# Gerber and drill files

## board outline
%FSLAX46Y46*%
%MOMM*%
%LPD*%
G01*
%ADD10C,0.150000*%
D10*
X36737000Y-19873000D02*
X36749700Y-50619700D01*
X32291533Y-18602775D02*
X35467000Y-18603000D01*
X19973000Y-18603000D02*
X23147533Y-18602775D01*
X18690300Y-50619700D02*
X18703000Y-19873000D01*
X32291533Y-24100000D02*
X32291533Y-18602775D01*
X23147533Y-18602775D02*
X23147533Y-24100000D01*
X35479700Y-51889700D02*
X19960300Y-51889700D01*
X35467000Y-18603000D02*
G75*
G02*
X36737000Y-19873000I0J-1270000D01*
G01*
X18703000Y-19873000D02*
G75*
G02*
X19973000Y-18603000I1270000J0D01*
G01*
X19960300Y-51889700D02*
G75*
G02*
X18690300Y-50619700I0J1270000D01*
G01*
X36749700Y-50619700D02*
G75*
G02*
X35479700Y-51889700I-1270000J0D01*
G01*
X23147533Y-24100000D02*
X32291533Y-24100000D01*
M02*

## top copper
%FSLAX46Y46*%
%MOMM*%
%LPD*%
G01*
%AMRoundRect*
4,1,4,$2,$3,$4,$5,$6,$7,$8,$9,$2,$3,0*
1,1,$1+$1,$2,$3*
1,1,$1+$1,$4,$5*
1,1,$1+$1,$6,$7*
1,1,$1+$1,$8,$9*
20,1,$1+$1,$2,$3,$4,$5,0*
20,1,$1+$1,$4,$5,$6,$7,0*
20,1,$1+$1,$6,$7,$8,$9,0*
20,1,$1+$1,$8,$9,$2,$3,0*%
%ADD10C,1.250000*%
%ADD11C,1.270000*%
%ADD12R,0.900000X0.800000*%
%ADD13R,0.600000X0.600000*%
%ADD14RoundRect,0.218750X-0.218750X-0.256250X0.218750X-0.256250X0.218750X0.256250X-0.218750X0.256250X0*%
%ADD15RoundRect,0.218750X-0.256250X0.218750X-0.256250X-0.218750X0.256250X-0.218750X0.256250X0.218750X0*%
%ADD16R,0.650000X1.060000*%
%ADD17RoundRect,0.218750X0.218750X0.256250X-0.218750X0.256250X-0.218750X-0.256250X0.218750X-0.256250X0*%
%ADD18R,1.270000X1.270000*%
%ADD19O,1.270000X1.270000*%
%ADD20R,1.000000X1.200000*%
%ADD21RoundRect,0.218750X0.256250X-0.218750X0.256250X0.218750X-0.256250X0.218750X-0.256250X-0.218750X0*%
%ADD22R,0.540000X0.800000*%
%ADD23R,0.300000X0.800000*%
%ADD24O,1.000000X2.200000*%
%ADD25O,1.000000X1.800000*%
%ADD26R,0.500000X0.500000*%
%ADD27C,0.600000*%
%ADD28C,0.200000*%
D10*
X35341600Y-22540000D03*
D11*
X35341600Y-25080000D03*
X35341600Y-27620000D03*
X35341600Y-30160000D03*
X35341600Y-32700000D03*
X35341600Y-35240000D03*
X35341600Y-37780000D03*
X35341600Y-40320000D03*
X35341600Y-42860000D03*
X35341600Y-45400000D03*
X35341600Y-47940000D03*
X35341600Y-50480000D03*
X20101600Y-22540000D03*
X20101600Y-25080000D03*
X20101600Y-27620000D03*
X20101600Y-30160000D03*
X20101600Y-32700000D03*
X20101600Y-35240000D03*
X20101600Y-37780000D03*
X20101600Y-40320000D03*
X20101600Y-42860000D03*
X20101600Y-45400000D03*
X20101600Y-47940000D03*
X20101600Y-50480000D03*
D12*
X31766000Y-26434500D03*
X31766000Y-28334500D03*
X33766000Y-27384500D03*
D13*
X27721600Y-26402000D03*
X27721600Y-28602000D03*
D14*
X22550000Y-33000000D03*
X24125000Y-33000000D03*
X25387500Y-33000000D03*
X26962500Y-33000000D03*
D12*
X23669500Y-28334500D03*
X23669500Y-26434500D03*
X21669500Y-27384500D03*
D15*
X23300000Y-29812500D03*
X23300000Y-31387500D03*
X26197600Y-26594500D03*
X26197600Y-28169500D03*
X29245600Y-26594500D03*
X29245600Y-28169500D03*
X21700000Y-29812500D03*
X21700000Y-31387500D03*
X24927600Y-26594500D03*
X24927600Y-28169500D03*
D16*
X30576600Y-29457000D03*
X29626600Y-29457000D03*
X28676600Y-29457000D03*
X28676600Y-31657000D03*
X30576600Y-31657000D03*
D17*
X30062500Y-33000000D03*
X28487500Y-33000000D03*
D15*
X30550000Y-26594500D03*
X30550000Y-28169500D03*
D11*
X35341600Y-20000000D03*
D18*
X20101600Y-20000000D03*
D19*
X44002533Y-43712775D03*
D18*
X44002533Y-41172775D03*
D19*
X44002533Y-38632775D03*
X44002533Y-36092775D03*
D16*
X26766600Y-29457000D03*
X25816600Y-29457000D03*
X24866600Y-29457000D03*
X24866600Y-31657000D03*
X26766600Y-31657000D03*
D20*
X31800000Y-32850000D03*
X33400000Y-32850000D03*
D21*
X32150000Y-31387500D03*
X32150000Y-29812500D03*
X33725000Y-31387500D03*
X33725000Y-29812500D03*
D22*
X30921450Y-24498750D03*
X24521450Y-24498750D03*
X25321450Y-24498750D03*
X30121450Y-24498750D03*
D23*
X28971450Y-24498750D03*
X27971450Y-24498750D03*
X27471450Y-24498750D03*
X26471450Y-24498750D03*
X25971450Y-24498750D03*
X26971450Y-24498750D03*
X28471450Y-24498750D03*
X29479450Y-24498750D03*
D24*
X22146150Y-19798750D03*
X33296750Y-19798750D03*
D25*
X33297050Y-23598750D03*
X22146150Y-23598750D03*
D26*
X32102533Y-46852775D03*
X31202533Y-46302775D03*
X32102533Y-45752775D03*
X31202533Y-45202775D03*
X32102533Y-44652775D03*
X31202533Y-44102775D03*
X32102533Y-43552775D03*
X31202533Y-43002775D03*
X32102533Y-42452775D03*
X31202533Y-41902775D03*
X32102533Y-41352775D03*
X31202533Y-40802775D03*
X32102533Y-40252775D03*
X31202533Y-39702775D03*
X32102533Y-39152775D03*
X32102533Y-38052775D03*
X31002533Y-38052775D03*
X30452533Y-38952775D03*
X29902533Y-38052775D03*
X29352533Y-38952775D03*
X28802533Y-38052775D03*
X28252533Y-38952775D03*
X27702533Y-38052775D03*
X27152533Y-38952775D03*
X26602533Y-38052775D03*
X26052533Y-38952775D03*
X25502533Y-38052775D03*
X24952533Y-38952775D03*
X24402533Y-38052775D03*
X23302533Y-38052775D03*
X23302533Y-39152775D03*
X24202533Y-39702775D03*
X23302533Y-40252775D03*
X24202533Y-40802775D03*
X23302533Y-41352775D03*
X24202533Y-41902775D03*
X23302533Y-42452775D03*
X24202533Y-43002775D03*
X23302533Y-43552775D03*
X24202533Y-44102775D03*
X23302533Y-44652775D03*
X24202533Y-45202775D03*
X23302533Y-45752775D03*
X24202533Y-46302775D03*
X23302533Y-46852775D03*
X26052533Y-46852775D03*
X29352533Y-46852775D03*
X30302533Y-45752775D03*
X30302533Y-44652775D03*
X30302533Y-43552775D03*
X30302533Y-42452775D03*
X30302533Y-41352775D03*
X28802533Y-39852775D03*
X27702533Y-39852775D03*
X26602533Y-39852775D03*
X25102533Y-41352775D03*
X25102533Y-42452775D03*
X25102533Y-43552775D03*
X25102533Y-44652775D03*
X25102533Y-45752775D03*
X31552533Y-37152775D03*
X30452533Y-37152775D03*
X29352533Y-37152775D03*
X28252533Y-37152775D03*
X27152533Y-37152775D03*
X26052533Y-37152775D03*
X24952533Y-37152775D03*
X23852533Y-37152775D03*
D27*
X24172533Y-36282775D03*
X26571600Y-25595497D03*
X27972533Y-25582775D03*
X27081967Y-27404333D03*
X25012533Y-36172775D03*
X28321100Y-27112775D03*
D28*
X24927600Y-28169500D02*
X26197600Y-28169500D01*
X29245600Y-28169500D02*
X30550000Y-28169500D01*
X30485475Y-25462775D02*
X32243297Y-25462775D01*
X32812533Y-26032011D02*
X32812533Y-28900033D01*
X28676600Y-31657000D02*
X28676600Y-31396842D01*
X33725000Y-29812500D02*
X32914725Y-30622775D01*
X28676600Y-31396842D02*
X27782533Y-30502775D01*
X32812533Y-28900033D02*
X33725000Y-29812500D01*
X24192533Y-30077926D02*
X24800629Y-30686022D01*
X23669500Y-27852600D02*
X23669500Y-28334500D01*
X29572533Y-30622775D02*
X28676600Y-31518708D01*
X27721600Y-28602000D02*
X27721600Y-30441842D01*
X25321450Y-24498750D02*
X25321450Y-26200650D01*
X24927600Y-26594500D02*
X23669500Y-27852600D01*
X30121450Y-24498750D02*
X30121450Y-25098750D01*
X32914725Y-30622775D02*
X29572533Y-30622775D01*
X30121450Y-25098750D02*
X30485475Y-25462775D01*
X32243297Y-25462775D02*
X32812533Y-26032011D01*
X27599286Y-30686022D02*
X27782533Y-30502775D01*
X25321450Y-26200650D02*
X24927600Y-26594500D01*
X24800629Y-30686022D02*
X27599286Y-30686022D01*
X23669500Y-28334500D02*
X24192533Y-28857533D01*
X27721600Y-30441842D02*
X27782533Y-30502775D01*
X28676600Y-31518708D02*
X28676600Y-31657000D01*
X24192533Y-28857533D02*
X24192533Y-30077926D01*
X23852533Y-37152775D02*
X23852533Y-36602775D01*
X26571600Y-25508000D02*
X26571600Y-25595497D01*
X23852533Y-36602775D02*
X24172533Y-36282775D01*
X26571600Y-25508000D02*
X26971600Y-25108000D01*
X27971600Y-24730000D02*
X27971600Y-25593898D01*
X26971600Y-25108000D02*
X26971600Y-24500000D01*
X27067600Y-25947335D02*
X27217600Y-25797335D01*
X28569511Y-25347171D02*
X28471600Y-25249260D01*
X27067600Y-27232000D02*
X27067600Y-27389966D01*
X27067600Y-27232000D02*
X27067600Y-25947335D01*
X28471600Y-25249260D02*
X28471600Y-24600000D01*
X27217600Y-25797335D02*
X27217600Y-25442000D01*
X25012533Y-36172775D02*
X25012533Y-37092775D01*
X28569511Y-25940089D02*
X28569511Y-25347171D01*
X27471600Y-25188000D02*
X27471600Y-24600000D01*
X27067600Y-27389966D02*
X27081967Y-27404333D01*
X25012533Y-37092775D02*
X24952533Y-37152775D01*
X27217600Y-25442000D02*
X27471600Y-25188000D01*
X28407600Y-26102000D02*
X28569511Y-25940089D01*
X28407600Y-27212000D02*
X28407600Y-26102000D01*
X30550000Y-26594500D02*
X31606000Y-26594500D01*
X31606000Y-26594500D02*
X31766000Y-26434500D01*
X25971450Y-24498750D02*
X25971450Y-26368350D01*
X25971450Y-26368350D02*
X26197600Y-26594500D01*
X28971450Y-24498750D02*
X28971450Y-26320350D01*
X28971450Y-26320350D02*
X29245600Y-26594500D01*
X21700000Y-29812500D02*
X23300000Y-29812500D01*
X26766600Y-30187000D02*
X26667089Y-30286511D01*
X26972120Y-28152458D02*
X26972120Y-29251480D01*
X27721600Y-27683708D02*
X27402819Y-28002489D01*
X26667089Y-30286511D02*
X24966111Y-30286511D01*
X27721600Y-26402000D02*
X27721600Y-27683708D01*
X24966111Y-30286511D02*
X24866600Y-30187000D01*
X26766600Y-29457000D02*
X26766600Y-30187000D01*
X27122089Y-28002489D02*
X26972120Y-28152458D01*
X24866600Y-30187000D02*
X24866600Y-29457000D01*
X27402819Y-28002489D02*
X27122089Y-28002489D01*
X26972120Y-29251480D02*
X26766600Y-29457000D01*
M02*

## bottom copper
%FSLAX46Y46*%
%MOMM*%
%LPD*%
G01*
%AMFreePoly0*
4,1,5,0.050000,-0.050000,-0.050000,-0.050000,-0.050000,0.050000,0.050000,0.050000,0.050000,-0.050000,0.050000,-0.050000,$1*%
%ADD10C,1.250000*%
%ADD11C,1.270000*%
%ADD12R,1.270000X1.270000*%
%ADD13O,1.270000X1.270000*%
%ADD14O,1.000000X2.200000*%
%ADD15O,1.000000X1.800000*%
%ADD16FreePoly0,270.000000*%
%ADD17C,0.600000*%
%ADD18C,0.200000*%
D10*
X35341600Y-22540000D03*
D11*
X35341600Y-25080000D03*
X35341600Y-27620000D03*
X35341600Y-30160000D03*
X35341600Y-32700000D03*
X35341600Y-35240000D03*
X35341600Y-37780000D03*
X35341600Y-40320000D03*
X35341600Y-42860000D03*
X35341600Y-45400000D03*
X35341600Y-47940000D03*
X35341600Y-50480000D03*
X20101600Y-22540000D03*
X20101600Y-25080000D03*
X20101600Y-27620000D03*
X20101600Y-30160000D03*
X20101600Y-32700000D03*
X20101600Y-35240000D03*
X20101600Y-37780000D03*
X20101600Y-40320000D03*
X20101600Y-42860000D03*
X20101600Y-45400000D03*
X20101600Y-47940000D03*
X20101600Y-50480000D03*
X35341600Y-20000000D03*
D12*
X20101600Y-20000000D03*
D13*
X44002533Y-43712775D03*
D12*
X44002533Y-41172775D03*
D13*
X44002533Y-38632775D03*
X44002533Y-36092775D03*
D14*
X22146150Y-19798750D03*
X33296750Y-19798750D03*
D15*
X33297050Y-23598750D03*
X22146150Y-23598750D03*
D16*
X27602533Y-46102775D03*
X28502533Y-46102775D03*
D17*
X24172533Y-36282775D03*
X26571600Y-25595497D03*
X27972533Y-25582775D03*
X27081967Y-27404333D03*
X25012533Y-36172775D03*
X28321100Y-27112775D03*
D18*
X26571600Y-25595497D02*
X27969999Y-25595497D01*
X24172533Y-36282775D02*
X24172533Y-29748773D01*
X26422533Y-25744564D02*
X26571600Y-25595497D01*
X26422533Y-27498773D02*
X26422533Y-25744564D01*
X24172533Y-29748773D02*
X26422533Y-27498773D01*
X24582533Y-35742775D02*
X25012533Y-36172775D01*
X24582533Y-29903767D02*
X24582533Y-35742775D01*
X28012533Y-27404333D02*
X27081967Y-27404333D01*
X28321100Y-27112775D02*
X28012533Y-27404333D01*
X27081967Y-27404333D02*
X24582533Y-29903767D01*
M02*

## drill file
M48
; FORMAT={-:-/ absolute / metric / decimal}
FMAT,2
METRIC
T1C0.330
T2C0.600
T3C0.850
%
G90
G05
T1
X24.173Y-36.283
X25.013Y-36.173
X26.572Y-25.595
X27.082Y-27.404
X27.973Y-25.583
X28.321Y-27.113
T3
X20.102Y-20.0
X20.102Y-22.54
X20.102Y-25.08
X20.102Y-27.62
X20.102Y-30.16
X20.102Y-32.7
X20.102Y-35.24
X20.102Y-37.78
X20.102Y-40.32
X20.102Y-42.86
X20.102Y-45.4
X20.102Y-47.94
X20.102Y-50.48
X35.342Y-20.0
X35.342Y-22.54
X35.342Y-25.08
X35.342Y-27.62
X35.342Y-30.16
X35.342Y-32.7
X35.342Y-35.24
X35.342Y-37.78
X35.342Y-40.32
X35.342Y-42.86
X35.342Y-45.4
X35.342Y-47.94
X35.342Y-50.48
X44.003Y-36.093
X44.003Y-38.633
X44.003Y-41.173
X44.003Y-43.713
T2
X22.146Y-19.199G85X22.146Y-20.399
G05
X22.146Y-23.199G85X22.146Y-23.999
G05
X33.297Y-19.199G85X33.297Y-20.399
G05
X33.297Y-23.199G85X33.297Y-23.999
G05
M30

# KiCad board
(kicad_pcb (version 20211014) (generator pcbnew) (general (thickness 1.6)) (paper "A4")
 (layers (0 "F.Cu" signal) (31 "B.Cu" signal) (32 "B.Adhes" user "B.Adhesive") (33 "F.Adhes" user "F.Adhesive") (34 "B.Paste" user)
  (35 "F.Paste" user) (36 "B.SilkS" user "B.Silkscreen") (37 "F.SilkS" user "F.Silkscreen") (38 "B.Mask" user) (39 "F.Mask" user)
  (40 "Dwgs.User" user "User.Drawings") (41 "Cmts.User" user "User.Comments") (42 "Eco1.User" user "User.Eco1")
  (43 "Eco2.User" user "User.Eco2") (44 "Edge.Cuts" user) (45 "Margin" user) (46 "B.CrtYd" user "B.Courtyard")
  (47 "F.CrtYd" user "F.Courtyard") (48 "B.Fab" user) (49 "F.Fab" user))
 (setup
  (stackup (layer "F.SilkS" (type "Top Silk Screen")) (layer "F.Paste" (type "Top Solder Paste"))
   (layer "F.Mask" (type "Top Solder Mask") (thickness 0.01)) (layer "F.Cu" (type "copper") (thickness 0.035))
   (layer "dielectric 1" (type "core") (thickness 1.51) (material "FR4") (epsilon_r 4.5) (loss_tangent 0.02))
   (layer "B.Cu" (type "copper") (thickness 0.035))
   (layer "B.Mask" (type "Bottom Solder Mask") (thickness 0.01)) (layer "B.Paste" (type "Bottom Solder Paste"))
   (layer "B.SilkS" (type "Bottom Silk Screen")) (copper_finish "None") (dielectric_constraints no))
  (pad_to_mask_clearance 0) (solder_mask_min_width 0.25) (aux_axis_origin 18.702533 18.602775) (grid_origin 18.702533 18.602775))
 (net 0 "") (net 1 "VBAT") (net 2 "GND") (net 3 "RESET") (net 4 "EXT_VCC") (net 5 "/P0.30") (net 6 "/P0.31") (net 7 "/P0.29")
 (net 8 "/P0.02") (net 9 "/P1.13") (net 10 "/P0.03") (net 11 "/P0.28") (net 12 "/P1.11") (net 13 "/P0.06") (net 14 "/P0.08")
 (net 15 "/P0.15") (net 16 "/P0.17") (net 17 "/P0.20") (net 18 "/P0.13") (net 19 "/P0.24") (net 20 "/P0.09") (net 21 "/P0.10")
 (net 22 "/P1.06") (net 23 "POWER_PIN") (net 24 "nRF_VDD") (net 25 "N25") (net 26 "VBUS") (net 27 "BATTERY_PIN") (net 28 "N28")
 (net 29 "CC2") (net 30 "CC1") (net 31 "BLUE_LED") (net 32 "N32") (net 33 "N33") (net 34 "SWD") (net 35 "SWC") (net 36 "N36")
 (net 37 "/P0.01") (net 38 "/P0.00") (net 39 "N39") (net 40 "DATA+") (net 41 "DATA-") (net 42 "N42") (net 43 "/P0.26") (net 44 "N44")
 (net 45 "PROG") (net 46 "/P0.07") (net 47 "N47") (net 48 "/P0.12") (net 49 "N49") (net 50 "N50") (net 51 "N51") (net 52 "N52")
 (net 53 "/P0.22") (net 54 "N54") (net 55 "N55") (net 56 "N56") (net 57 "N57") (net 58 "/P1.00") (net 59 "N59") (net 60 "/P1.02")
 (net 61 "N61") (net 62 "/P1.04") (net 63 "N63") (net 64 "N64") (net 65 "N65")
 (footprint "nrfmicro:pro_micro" (layer "F.Cu") (at 27.7216 36.51)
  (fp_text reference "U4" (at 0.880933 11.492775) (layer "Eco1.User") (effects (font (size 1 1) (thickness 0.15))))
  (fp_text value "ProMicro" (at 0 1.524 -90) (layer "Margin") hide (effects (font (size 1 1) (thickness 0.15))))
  (pad "1" thru_hole circle locked (at 7.62 -13.97 270) (size 1.25 1.25) (drill 0.85) (layers *.Cu *.Mask) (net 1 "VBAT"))
  (pad "2" thru_hole circle locked (at 7.62 -11.43 270) (size 1.27 1.27) (drill 0.85) (layers *.Cu *.Mask) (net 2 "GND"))
  (pad "3" thru_hole circle locked (at 7.62 -8.89 270) (size 1.27 1.27) (drill 0.85) (layers *.Cu *.Mask) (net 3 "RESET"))
  (pad "4" thru_hole circle locked (at 7.62 -6.35 270) (size 1.27 1.27) (drill 0.85) (layers *.Cu *.Mask) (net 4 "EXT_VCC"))
  (pad "5" thru_hole circle locked (at 7.62 -3.81 270) (size 1.27 1.27) (drill 0.85) (layers *.Cu *.Mask) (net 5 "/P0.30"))
  (pad "6" thru_hole circle locked (at 7.62 -1.27 270) (size 1.27 1.27) (drill 0.85) (layers *.Cu *.Mask) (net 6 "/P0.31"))
  (pad "7" thru_hole circle locked (at 7.62 1.27 270) (size 1.27 1.27) (drill 0.85) (layers *.Cu *.Mask) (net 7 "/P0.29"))
  (pad "8" thru_hole circle locked (at 7.62 3.81 270) (size 1.27 1.27) (drill 0.85) (layers *.Cu *.Mask) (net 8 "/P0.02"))
  (pad "9" thru_hole circle locked (at 7.62 6.35 270) (size 1.27 1.27) (drill 0.85) (layers *.Cu *.Mask) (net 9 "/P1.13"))
  (pad "10" thru_hole circle locked (at 7.62 8.89 270) (size 1.27 1.27) (drill 0.85) (layers *.Cu *.Mask) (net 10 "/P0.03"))
  (pad "11" thru_hole circle locked (at 7.62 11.43 270) (size 1.27 1.27) (drill 0.85) (layers *.Cu *.Mask) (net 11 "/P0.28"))
  (pad "12" thru_hole circle locked (at 7.62 13.97 270) (size 1.27 1.27) (drill 0.85) (layers *.Cu *.Mask) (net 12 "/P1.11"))
  (pad "13" thru_hole circle locked (at -7.62 -13.97 270) (size 1.27 1.27) (drill 0.85) (layers *.Cu *.Mask) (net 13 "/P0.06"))
  (pad "14" thru_hole circle locked (at -7.62 -11.43 270) (size 1.27 1.27) (drill 0.85) (layers *.Cu *.Mask) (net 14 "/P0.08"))
  (pad "15" thru_hole circle locked (at -7.62 -8.89 270) (size 1.27 1.27) (drill 0.85) (layers *.Cu *.Mask) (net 2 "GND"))
  (pad "16" thru_hole circle locked (at -7.62 -6.35 270) (size 1.27 1.27) (drill 0.85) (layers *.Cu *.Mask) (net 2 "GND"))
  (pad "17" thru_hole circle locked (at -7.62 -3.81 270) (size 1.27 1.27) (drill 0.85) (layers *.Cu *.Mask) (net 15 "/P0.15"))
  (pad "18" thru_hole circle locked (at -7.62 -1.27 270) (size 1.27 1.27) (drill 0.85) (layers *.Cu *.Mask) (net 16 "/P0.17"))
  (pad "19" thru_hole circle locked (at -7.62 1.27 270) (size 1.27 1.27) (drill 0.85) (layers *.Cu *.Mask) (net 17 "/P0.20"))
  (pad "20" thru_hole circle locked (at -7.62 3.81 270) (size 1.27 1.27) (drill 0.85) (layers *.Cu *.Mask) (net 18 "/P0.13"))
  (pad "21" thru_hole circle locked (at -7.62 6.35 270) (size 1.27 1.27) (drill 0.85) (layers *.Cu *.Mask) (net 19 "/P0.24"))
  (pad "22" thru_hole circle locked (at -7.62 8.89 270) (size 1.27 1.27) (drill 0.85) (layers *.Cu *.Mask) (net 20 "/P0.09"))
  (pad "23" thru_hole circle locked (at -7.62 11.43 270) (size 1.27 1.27) (drill 0.85) (layers *.Cu *.Mask) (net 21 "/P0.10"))
  (pad "24" thru_hole circle locked (at -7.62 13.97 270) (size 1.27 1.27) (drill 0.85) (layers *.Cu *.Mask) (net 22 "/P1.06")))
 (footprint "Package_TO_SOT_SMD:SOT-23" (layer "F.Cu") (at 32.766 27.3845)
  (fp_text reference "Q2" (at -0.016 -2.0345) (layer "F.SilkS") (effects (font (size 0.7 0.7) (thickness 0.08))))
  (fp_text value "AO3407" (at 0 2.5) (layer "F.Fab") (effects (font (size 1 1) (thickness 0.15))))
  (pad "1" smd rect locked (at -1 -0.95) (size 0.9 0.8) (layers "F.Cu" "F.Paste" "F.Mask") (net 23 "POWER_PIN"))
  (pad "2" smd rect locked (at -1 0.95) (size 0.9 0.8) (layers "F.Cu" "F.Paste" "F.Mask") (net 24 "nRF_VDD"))
  (pad "3" smd rect locked (at 1 0) (size 0.9 0.8) (layers "F.Cu" "F.Paste" "F.Mask") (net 4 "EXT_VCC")))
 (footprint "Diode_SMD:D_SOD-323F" (layer "F.Cu") (at 27.7216 27.502 -90)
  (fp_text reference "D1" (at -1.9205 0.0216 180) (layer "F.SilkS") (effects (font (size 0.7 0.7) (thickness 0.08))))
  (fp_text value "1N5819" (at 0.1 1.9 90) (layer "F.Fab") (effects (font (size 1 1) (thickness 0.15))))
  (pad "1" smd rect locked (at -1.1 0 270) (size 0.6 0.6) (layers "F.Cu" "F.Paste" "F.Mask") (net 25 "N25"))
  (pad "2" smd rect locked (at 1.1 0 270) (size 0.6 0.6) (layers "F.Cu" "F.Paste" "F.Mask") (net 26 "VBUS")))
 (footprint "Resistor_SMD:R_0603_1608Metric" (layer "F.Cu") (at 23.3375 33)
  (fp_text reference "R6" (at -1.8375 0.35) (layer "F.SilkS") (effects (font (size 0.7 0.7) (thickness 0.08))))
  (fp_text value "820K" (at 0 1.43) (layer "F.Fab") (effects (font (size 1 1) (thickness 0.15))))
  (pad "1" smd roundrect locked (at -0.7875 0) (size 0.875 0.95) (layers "F.Cu" "F.Paste" "F.Mask") (roundrect_rratio 0.25) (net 1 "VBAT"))
  (pad "2" smd roundrect locked (at 0.7875 0) (size 0.875 0.95) (layers "F.Cu" "F.Paste" "F.Mask") (roundrect_rratio 0.25)
   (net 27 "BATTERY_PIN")))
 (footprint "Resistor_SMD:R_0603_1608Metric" (layer "F.Cu") (at 26.175 33)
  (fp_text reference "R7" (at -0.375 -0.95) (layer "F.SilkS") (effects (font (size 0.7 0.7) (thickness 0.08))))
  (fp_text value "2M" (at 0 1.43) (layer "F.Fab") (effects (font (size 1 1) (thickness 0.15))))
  (pad "1" smd roundrect locked (at -0.7875 0) (size 0.875 0.95) (layers "F.Cu" "F.Paste" "F.Mask") (roundrect_rratio 0.25)
   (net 27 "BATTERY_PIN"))
  (pad "2" smd roundrect locked (at 0.7875 0) (size 0.875 0.95) (layers "F.Cu" "F.Paste" "F.Mask") (roundrect_rratio 0.25) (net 2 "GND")))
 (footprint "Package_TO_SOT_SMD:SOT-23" (layer "F.Cu") (at 22.6695 27.3845 180)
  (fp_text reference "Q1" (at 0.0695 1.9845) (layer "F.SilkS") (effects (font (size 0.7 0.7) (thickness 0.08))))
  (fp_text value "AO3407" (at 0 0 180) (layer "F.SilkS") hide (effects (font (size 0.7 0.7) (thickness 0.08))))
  (pad "1" smd rect locked (at -1 -0.95 180) (size 0.9 0.8) (layers "F.Cu" "F.Paste" "F.Mask") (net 26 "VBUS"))
  (pad "2" smd rect locked (at -1 0.95 180) (size 0.9 0.8) (layers "F.Cu" "F.Paste" "F.Mask") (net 25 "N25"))
  (pad "3" smd rect locked (at 1 0 180) (size 0.9 0.8) (layers "F.Cu" "F.Paste" "F.Mask") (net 1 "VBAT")))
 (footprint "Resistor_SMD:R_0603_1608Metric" (layer "F.Cu") (at 23.3 30.6 -90)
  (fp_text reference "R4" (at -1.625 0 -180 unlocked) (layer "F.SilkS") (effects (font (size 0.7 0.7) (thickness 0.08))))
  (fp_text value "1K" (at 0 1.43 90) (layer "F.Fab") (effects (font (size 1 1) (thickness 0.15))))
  (pad "1" smd roundrect locked (at -0.7875 0 270) (size 0.875 0.95) (layers "F.Cu" "F.Paste" "F.Mask") (roundrect_rratio 0.25)
   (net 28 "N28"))
  (pad "2" smd roundrect locked (at 0.7875 0 270) (size 0.875 0.95) (layers "F.Cu" "F.Paste" "F.Mask") (roundrect_rratio 0.25) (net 2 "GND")))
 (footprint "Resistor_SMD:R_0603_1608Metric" (layer "F.Cu") (at 26.1976 27.382 -90)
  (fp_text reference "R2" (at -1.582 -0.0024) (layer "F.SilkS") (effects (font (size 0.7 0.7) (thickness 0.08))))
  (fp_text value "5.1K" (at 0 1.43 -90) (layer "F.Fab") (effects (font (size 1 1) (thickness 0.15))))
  (pad "1" smd roundrect locked (at -0.7875 0 270) (size 0.875 0.95) (layers "F.Cu" "F.Paste" "F.Mask") (roundrect_rratio 0.25)
   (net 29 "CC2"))
  (pad "2" smd roundrect locked (at 0.7875 0 270) (size 0.875 0.95) (layers "F.Cu" "F.Paste" "F.Mask") (roundrect_rratio 0.25) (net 2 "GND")))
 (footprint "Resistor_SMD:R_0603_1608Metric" (layer "F.Cu") (at 29.2456 27.382 -90)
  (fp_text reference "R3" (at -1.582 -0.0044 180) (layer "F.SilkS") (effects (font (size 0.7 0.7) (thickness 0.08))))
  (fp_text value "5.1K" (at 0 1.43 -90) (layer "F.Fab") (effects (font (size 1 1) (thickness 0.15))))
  (pad "1" smd roundrect locked (at -0.7875 0 270) (size 0.875 0.95) (layers "F.Cu" "F.Paste" "F.Mask") (roundrect_rratio 0.25)
   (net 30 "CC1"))
  (pad "2" smd roundrect locked (at 0.7875 0 270) (size 0.875 0.95) (layers "F.Cu" "F.Paste" "F.Mask") (roundrect_rratio 0.25) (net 2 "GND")))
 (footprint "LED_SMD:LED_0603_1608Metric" (layer "F.Cu") (at 21.7 30.6 -90)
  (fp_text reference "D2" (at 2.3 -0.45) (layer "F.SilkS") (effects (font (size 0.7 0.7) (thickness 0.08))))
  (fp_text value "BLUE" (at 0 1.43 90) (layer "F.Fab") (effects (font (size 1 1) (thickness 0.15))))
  (pad "1" smd roundrect locked (at -0.7875 0 270) (size 0.875 0.95) (layers "F.Cu" "F.Paste" "F.Mask") (roundrect_rratio 0.25)
   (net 28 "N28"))
  (pad "2" smd roundrect locked (at 0.7875 0 270) (size 0.875 0.95) (layers "F.Cu" "F.Paste" "F.Mask") (roundrect_rratio 0.25)
   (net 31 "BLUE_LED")))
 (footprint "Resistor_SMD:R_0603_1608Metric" (layer "F.Cu") (at 24.9276 27.382 -90)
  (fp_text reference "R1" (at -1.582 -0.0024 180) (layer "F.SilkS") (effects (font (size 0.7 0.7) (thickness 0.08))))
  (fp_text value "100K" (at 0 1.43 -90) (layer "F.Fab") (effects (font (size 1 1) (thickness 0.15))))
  (pad "1" smd roundrect locked (at -0.7875 0 270) (size 0.875 0.95) (layers "F.Cu" "F.Paste" "F.Mask") (roundrect_rratio 0.25)
   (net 26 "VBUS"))
  (pad "2" smd roundrect locked (at 0.7875 0 270) (size 0.875 0.95) (layers "F.Cu" "F.Paste" "F.Mask") (roundrect_rratio 0.25) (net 2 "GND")))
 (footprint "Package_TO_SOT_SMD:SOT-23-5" (layer "F.Cu") (at 29.6266 30.557 -90)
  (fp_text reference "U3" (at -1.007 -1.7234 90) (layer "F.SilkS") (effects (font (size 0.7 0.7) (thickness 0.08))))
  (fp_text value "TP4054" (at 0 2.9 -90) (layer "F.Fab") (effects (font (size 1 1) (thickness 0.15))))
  (pad "1" smd rect locked (at -1.1 -0.95 270) (size 1.06 0.65) (layers "F.Cu" "F.Paste" "F.Mask") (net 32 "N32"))
  (pad "2" smd rect locked (at -1.1 0 270) (size 1.06 0.65) (layers "F.Cu" "F.Paste" "F.Mask") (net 2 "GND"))
  (pad "3" smd rect locked (at -1.1 0.95 270) (size 1.06 0.65) (layers "F.Cu" "F.Paste" "F.Mask") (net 1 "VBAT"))
  (pad "4" smd rect locked (at 1.1 0.95 270) (size 1.06 0.65) (layers "F.Cu" "F.Paste" "F.Mask") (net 26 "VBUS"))
  (pad "5" smd rect locked (at 1.1 -0.95 270) (size 1.06 0.65) (layers "F.Cu" "F.Paste" "F.Mask") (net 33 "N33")))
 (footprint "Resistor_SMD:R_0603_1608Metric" (layer "F.Cu") (at 29.275 33 180)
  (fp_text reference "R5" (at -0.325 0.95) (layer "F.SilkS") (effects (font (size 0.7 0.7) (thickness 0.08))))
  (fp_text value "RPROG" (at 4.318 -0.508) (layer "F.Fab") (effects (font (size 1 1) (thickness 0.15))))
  (pad "1" smd roundrect locked (at -0.7875 0 180) (size 0.875 0.95) (layers "F.Cu" "F.Paste" "F.Mask") (roundrect_rratio 0.25)
   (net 33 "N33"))
  (pad "2" smd roundrect locked (at 0.7875 0 180) (size 0.875 0.95) (layers "F.Cu" "F.Paste" "F.Mask") (roundrect_rratio 0.25) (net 2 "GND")))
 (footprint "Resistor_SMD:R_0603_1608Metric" (layer "F.Cu") (at 30.55 27.382 -90)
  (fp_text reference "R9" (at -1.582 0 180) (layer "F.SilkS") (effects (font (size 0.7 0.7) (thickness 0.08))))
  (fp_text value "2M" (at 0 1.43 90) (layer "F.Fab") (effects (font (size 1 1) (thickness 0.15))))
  (pad "1" smd roundrect locked (at -0.7875 0 270) (size 0.875 0.95) (layers "F.Cu" "F.Paste" "F.Mask") (roundrect_rratio 0.25)
   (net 23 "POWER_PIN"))
  (pad "2" smd roundrect locked (at 0.7875 0 270) (size 0.875 0.95) (layers "F.Cu" "F.Paste" "F.Mask") (roundrect_rratio 0.25) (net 2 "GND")))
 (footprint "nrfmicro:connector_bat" (layer "F.Cu") (at 27.7216 20 180)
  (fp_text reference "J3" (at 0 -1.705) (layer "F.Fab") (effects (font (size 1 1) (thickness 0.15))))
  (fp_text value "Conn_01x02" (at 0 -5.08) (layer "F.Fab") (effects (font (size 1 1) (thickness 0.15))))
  (pad "1" thru_hole circle locked (at -7.62 0 270) (size 1.27 1.27) (drill 0.85) (layers *.Cu *.Mask) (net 1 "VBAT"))
  (pad "2" thru_hole rect locked (at 7.62 0 180) (size 1.27 1.27) (drill 0.85) (layers *.Cu *.Mask) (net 2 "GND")))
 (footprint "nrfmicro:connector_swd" (layer "F.Cu") (at 44.002533 43.712775 180)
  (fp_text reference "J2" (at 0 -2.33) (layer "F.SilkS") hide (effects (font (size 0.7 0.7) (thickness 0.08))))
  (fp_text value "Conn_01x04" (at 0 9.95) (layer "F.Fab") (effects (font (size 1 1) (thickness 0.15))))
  (pad "1" thru_hole oval locked (at 0 0 180) (size 1.27 1.27) (drill 0.85) (layers *.Cu *.Mask) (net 24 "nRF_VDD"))
  (pad "2" thru_hole rect locked (at 0 2.54 180) (size 1.27 1.27) (drill 0.85) (layers *.Cu *.Mask) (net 2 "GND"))
  (pad "3" thru_hole oval locked (at 0 5.08 180) (size 1.27 1.27) (drill 0.85) (layers *.Cu *.Mask) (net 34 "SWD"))
  (pad "4" thru_hole oval locked (at 0 7.62 180) (size 1.27 1.27) (drill 0.85) (layers *.Cu *.Mask) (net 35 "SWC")))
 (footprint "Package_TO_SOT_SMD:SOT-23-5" (layer "F.Cu") (at 25.8166 30.557 -90)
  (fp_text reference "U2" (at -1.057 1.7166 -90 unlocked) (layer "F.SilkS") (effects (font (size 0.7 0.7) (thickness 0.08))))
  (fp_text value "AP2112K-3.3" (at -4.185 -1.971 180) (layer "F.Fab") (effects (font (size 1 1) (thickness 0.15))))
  (pad "1" smd rect locked (at -1.1 -0.95 270) (size 1.06 0.65) (layers "F.Cu" "F.Paste" "F.Mask") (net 25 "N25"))
  (pad "2" smd rect locked (at -1.1 0 270) (size 1.06 0.65) (layers "F.Cu" "F.Paste" "F.Mask") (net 2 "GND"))
  (pad "3" smd rect locked (at -1.1 0.95 270) (size 1.06 0.65) (layers "F.Cu" "F.Paste" "F.Mask") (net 25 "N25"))
  (pad "4" smd rect locked (at 1.1 0.95 270) (size 1.06 0.65) (layers "F.Cu" "F.Paste" "F.Mask") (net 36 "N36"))
  (pad "5" smd rect locked (at 1.1 -0.95 270) (size 1.06 0.65) (layers "F.Cu" "F.Paste" "F.Mask") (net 24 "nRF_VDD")))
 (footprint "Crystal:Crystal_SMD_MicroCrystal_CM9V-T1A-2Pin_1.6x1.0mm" (layer "F.Cu") (at 32.6 32.85)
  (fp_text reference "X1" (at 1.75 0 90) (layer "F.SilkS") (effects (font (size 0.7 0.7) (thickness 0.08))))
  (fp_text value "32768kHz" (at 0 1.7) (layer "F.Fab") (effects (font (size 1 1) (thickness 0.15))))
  (pad "1" smd rect locked (at -0.8 0) (size 1 1.2) (layers "F.Cu" "F.Paste" "F.Mask") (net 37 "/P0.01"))
  (pad "2" smd rect locked (at 0.8 0) (size 1 1.2) (layers "F.Cu" "F.Paste" "F.Mask") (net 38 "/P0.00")))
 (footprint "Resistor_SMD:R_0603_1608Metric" (layer "F.Cu") (at 32.15 30.6 90)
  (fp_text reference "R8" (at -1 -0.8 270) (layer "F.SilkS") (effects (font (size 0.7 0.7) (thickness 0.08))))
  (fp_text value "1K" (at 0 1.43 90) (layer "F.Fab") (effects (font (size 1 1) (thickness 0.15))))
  (pad "1" smd roundrect locked (at -0.7875 0 90) (size 0.875 0.95) (layers "F.Cu" "F.Paste" "F.Mask") (roundrect_rratio 0.25)
   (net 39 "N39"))
  (pad "2" smd roundrect locked (at 0.7875 0 90) (size 0.875 0.95) (layers "F.Cu" "F.Paste" "F.Mask") (roundrect_rratio 0.25) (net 32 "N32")))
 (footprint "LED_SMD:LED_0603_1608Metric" (layer "F.Cu") (at 33.725 30.6 90)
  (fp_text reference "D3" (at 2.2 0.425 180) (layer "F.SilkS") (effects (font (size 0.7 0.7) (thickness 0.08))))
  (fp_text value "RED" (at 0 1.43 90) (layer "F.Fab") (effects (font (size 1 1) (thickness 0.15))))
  (pad "1" smd roundrect locked (at -0.7875 0 90) (size 0.875 0.95) (layers "F.Cu" "F.Paste" "F.Mask") (roundrect_rratio 0.25)
   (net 39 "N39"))
  (pad "2" smd roundrect locked (at 0.7875 0 90) (size 0.875 0.95) (layers "F.Cu" "F.Paste" "F.Mask") (roundrect_rratio 0.25)
   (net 26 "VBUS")))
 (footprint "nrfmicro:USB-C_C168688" (layer "F.Cu") (at 27.72645 24.09875)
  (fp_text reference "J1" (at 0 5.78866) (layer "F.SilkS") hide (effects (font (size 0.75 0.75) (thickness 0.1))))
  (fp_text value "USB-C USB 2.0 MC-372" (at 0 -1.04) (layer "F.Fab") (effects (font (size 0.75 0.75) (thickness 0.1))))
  (pad "A1" smd rect (at 3.195 0.4) (size 0.54 0.8) (layers "F.Cu" "F.Paste" "F.Mask") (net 2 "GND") (clearance 0.15))
  (pad "A1" smd rect (at -3.205 0.4) (size 0.54 0.8) (layers "F.Cu" "F.Paste" "F.Mask") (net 2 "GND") (clearance 0.15))
  (pad "A4" smd rect (at -2.405 0.4) (size 0.54 0.8) (layers "F.Cu" "F.Paste" "F.Mask") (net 26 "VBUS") (clearance 0.15))
  (pad "A4" smd rect (at 2.395 0.4) (size 0.54 0.8) (layers "F.Cu" "F.Paste" "F.Mask") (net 26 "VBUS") (clearance 0.15))
  (pad "A5" smd rect (at 1.245 0.4) (size 0.3 0.8) (layers "F.Cu" "F.Paste" "F.Mask") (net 30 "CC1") (clearance 0.15))
  (pad "A6" smd rect (at 0.245 0.4) (size 0.3 0.8) (layers "F.Cu" "F.Paste" "F.Mask") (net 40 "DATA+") (clearance 0.15))
  (pad "A7" smd rect (at -0.255 0.4) (size 0.3 0.8) (layers "F.Cu" "F.Paste" "F.Mask") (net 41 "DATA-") (clearance 0.15))
  (pad "A8" smd rect (at -1.255 0.4) (size 0.3 0.8) (layers "F.Cu" "F.Paste" "F.Mask") (clearance 0.15))
  (pad "B5" smd rect (at -1.755 0.4) (size 0.3 0.8) (layers "F.Cu" "F.Paste" "F.Mask") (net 29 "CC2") (clearance 0.15))
  (pad "B6" smd rect (at -0.755 0.4) (size 0.3 0.8) (layers "F.Cu" "F.Paste" "F.Mask") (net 40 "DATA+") (clearance 0.15))
  (pad "B7" smd rect (at 0.745 0.4) (size 0.3 0.8) (layers "F.Cu" "F.Paste" "F.Mask") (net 41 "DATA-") (clearance 0.15))
  (pad "B8" smd rect (at 1.753 0.4) (size 0.3 0.8) (layers "F.Cu" "F.Paste" "F.Mask") (clearance 0.15))
  (pad "S1" thru_hole oval (at -5.5803 -4.3) (size 1 2.2) (drill oval 0.6 1.8) (layers *.Cu *.Mask "F.Paste") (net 2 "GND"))
  (pad "S1" thru_hole oval (at 5.5703 -4.3) (size 1 2.2) (drill oval 0.6 1.8) (layers *.Cu *.Mask "F.Paste") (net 2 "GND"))
  (pad "S1" thru_hole oval (at 5.5706 -0.5) (size 1 1.8) (drill oval 0.6 1.4) (layers *.Cu *.Mask "F.Paste") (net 2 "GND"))
  (pad "S1" thru_hole oval (at -5.5803 -0.5) (size 1 1.8) (drill oval 0.6 1.4) (layers *.Cu *.Mask "F.Paste") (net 2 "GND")))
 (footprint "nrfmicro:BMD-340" (layer "F.Cu") (at 27.702533 44.002775 90)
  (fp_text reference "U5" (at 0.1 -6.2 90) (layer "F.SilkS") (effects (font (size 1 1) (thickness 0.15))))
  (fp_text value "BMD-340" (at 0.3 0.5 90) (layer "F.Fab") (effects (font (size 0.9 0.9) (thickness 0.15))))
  (pad "1" smd rect locked (at -2.85 4.4 90) (size 0.5 0.5) (layers "F.Cu" "F.Paste" "F.Mask") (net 2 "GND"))
  (pad "2" smd rect locked (at -2.3 3.5 90) (size 0.5 0.5) (layers "F.Cu" "F.Paste" "F.Mask") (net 2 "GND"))
  (pad "3" smd rect locked (at -1.75 4.4 90) (size 0.5 0.5) (layers "F.Cu" "F.Paste" "F.Mask") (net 2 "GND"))
  (pad "4" smd rect locked (at -1.2 3.5 90) (size 0.5 0.5) (layers "F.Cu" "F.Paste" "F.Mask") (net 2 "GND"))
  (pad "5" smd rect locked (at -0.65 4.4 90) (size 0.5 0.5) (layers "F.Cu" "F.Paste" "F.Mask") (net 2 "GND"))
  (pad "6" smd rect locked (at -0.1 3.5 90) (size 0.5 0.5) (layers "F.Cu" "F.Paste" "F.Mask") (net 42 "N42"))
  (pad "7" smd rect locked (at 0.45 4.4 90) (size 0.5 0.5) (layers "F.Cu" "F.Paste" "F.Mask") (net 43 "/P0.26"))
  (pad "8" smd rect locked (at 1 3.5 90) (size 0.5 0.5) (layers "F.Cu" "F.Paste" "F.Mask") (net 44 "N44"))
  (pad "9" smd rect locked (at 1.55 4.4 90) (size 0.5 0.5) (layers "F.Cu" "F.Paste" "F.Mask") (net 11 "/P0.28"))
  (pad "10" smd rect locked (at 2.1 3.5 90) (size 0.5 0.5) (layers "F.Cu" "F.Paste" "F.Mask") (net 7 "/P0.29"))
  (pad "11" smd rect locked (at 2.65 4.4 90) (size 0.5 0.5) (layers "F.Cu" "F.Paste" "F.Mask") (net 5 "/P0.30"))
  (pad "12" smd rect locked (at 3.2 3.5 90) (size 0.5 0.5) (layers "F.Cu" "F.Paste" "F.Mask") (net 6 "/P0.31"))
  (pad "13" smd rect locked (at 3.75 4.4 90) (size 0.5 0.5) (layers "F.Cu" "F.Paste" "F.Mask") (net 38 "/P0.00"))
  (pad "14" smd rect locked (at 4.3 3.5 90) (size 0.5 0.5) (layers "F.Cu" "F.Paste" "F.Mask") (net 37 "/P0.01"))
  (pad "15" smd rect locked (at 4.85 4.4 90) (size 0.5 0.5) (layers "F.Cu" "F.Paste" "F.Mask") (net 8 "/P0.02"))
  (pad "16" smd rect locked (at 5.95 4.4 90) (size 0.5 0.5) (layers "F.Cu" "F.Paste" "F.Mask") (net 2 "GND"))
  (pad "17" smd rect locked (at 5.95 3.3 90) (size 0.5 0.5) (layers "F.Cu" "F.Paste" "F.Mask") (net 24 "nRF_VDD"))
  (pad "18" smd rect locked (at 5.05 2.75 90) (size 0.5 0.5) (layers "F.Cu" "F.Paste" "F.Mask") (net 2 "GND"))
  (pad "19" smd rect locked (at 5.95 2.2 90) (size 0.5 0.5) (layers "F.Cu" "F.Paste" "F.Mask") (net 10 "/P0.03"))
  (pad "20" smd rect locked (at 5.05 1.65 90) (size 0.5 0.5) (layers "F.Cu" "F.Paste" "F.Mask") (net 27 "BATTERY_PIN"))
  (pad "21" smd rect locked (at 5.95 1.1 90) (size 0.5 0.5) (layers "F.Cu" "F.Paste" "F.Mask") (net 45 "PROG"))
  (pad "22" smd rect locked (at 5.05 0.55 90) (size 0.5 0.5) (layers "F.Cu" "F.Paste" "F.Mask") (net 13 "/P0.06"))
  (pad "23" smd rect locked (at 5.95 0 90) (size 0.5 0.5) (layers "F.Cu" "F.Paste" "F.Mask") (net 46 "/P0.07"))
  (pad "24" smd rect locked (at 5.05 -0.55 90) (size 0.5 0.5) (layers "F.Cu" "F.Paste" "F.Mask") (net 14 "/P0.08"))
  (pad "25" smd rect locked (at 5.95 -1.1 90) (size 0.5 0.5) (layers "F.Cu" "F.Paste" "F.Mask") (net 20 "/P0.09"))
  (pad "26" smd rect locked (at 5.05 -1.65 90) (size 0.5 0.5) (layers "F.Cu" "F.Paste" "F.Mask") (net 21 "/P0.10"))
  (pad "27" smd rect locked (at 5.95 -2.2 90) (size 0.5 0.5) (layers "F.Cu" "F.Paste" "F.Mask") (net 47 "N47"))
  (pad "28" smd rect locked (at 5.05 -2.75 90) (size 0.5 0.5) (layers "F.Cu" "F.Paste" "F.Mask") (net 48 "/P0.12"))
  (pad "29" smd rect locked (at 5.95 -3.3 90) (size 0.5 0.5) (layers "F.Cu" "F.Paste" "F.Mask") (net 2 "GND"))
  (pad "30" smd rect locked (at 5.95 -4.4 90) (size 0.5 0.5) (layers "F.Cu" "F.Paste" "F.Mask") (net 2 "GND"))
  (pad "31" smd rect locked (at 4.85 -4.4 90) (size 0.5 0.5) (layers "F.Cu" "F.Paste" "F.Mask") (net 18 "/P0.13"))
  (pad "32" smd rect locked (at 4.3 -3.5 90) (size 0.5 0.5) (layers "F.Cu" "F.Paste" "F.Mask") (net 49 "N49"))
  (pad "33" smd rect locked (at 3.75 -4.4 90) (size 0.5 0.5) (layers "F.Cu" "F.Paste" "F.Mask") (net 15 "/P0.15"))
  (pad "34" smd rect locked (at 3.2 -3.5 90) (size 0.5 0.5) (layers "F.Cu" "F.Paste" "F.Mask") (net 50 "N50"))
  (pad "35" smd rect locked (at 2.65 -4.4 90) (size 0.5 0.5) (layers "F.Cu" "F.Paste" "F.Mask") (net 16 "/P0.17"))
  (pad "36" smd rect locked (at 2.1 -3.5 90) (size 0.5 0.5) (layers "F.Cu" "F.Paste" "F.Mask") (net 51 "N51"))
  (pad "37" smd rect locked (at 1.55 -4.4 90) (size 0.5 0.5) (layers "F.Cu" "F.Paste" "F.Mask") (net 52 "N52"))
  (pad "38" smd rect locked (at 1 -3.5 90) (size 0.5 0.5) (layers "F.Cu" "F.Paste" "F.Mask") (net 17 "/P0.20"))
  (pad "39" smd rect locked (at 0.45 -4.4 90) (size 0.5 0.5) (layers "F.Cu" "F.Paste" "F.Mask") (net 3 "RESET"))
  (pad "40" smd rect locked (at -0.1 -3.5 90) (size 0.5 0.5) (layers "F.Cu" "F.Paste" "F.Mask") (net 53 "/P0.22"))
  (pad "41" smd rect locked (at -0.65 -4.4 90) (size 0.5 0.5) (layers "F.Cu" "F.Paste" "F.Mask") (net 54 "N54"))
  (pad "42" smd rect locked (at -1.2 -3.5 90) (size 0.5 0.5) (layers "F.Cu" "F.Paste" "F.Mask") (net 19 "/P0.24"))
  (pad "43" smd rect locked (at -1.75 -4.4 90) (size 0.5 0.5) (layers "F.Cu" "F.Paste" "F.Mask") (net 35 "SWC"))
  (pad "44" smd rect locked (at -2.3 -3.5 90) (size 0.5 0.5) (layers "F.Cu" "F.Paste" "F.Mask") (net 34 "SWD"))
  (pad "45" smd rect locked (at -2.85 -4.4 90) (size 0.5 0.5) (layers "F.Cu" "F.Paste" "F.Mask") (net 2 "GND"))
  (pad "46" smd rect locked (at -2.85 -1.65 90) (size 0.5 0.5) (layers "F.Cu" "F.Paste" "F.Mask") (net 2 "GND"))
  (pad "47" smd rect locked (at -2.85 1.65 90) (size 0.5 0.5) (layers "F.Cu" "F.Paste" "F.Mask") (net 2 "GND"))
  (pad "48" smd rect locked (at -1.75 2.6 90) (size 0.5 0.5) (layers "F.Cu" "F.Paste" "F.Mask") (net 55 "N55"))
  (pad "49" smd rect locked (at -0.65 2.6 90) (size 0.5 0.5) (layers "F.Cu" "F.Paste" "F.Mask") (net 22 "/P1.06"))
  (pad "50" smd rect locked (at 0.45 2.6 90) (size 0.5 0.5) (layers "F.Cu" "F.Paste" "F.Mask") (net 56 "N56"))
  (pad "51" smd rect locked (at 1.55 2.6 90) (size 0.5 0.5) (layers "F.Cu" "F.Paste" "F.Mask") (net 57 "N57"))
  (pad "52" smd rect locked (at 2.65 2.6 90) (size 0.5 0.5) (layers "F.Cu" "F.Paste" "F.Mask") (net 23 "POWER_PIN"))
  (pad "53" smd rect locked (at 4.15 1.1 90) (size 0.5 0.5) (layers "F.Cu" "F.Paste" "F.Mask") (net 31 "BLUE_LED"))
  (pad "54" smd rect locked (at 4.15 0 90) (size 0.5 0.5) (layers "F.Cu" "F.Paste" "F.Mask") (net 12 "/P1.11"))
  (pad "55" smd rect locked (at 4.15 -1.1 90) (size 0.5 0.5) (layers "F.Cu" "F.Paste" "F.Mask") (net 2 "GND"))
  (pad "56" smd rect locked (at 2.65 -2.6 90) (size 0.5 0.5) (layers "F.Cu" "F.Paste" "F.Mask") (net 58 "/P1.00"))
  (pad "57" smd rect locked (at 1.55 -2.6 90) (size 0.5 0.5) (layers "F.Cu" "F.Paste" "F.Mask") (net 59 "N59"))
  (pad "58" smd rect locked (at 0.45 -2.6 90) (size 0.5 0.5) (layers "F.Cu" "F.Paste" "F.Mask") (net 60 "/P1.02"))
  (pad "59" smd rect locked (at -0.65 -2.6 90) (size 0.5 0.5) (layers "F.Cu" "F.Paste" "F.Mask") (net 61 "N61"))
  (pad "60" smd rect locked (at -1.75 -2.6 90) (size 0.5 0.5) (layers "F.Cu" "F.Paste" "F.Mask") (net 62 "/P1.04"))
  (pad "61" smd rect locked (at 6.85 3.85 90) (size 0.5 0.5) (layers "F.Cu" "F.Paste" "F.Mask") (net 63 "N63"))
  (pad "62" smd rect locked (at 6.85 2.75 90) (size 0.5 0.5) (layers "F.Cu" "F.Paste" "F.Mask") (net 9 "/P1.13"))
  (pad "63" smd rect locked (at 6.85 1.65 90) (size 0.5 0.5) (layers "F.Cu" "F.Paste" "F.Mask") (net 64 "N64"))
  (pad "64" smd rect locked (at 6.85 0.55 90) (size 0.5 0.5) (layers "F.Cu" "F.Paste" "F.Mask") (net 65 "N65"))
  (pad "65" smd rect locked (at 6.85 -0.55 90) (size 0.5 0.5) (layers "F.Cu" "F.Paste" "F.Mask") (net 24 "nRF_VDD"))
  (pad "66" smd rect locked (at 6.85 -1.65 90) (size 0.5 0.5) (layers "F.Cu" "F.Paste" "F.Mask") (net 26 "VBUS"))
  (pad "67" smd rect locked (at 6.85 -2.75 90) (size 0.5 0.5) (layers "F.Cu" "F.Paste" "F.Mask") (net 41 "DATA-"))
  (pad "68" smd rect locked (at 6.85 -3.85 90) (size 0.5 0.5) (layers "F.Cu" "F.Paste" "F.Mask") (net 40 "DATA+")))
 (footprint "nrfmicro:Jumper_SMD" (layer "B.Cu") (at 27.702533 46.102775 -90)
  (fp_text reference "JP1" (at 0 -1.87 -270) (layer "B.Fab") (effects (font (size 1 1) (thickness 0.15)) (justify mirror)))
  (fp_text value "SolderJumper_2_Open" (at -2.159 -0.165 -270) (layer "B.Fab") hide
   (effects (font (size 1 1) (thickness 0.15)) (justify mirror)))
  (pad "1" smd custom locked (at 0 0.1 270) (size 0.1 0.1) (layers "B.Cu" "B.Mask") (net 62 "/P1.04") (clearance 0.14) (zone_connect 0)
   (options (clearance outline) (anchor rect)) (primitives))
  (pad "2" smd custom locked (at 0 -0.8 270) (size 0.1 0.1) (layers "B.Cu" "B.Mask") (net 12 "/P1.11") (clearance 0.14) (zone_connect 0)
   (options (clearance outline) (anchor rect)) (primitives)))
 (gr_line (start 36.737 19.873) (end 36.7497 50.6197) (layer "Edge.Cuts") (width 0.15))
 (gr_line (start 32.291533 18.602775) (end 35.467 18.603) (layer "Edge.Cuts") (width 0.15))
 (gr_line (start 19.973 18.603) (end 23.147533 18.602775) (layer "Edge.Cuts") (width 0.15))
 (gr_line (start 18.6903 50.6197) (end 18.703 19.873) (layer "Edge.Cuts") (width 0.15))
 (gr_line (start 32.291533 24.1) (end 32.291533 18.602775) (layer "Edge.Cuts") (width 0.15))
 (gr_line (start 23.147533 18.602775) (end 23.147533 24.1) (layer "Edge.Cuts") (width 0.15))
 (gr_line (start 35.4797 51.8897) (end 19.9603 51.8897) (layer "Edge.Cuts") (width 0.15))
 (gr_arc (start 35.467 18.603) (mid 36.365026 18.974974) (end 36.737 19.873) (layer "Edge.Cuts") (width 0.15))
 (gr_arc (start 18.703 19.873) (mid 19.074974 18.974974) (end 19.973 18.603) (layer "Edge.Cuts") (width 0.15))
 (gr_arc (start 19.9603 51.8897) (mid 19.062274 51.517726) (end 18.6903 50.6197) (layer "Edge.Cuts") (width 0.15))
 (gr_arc (start 36.7497 50.6197) (mid 36.377726 51.517726) (end 35.4797 51.8897) (layer "Edge.Cuts") (width 0.15))
 (gr_line (start 23.147533 24.1) (end 32.291533 24.1) (layer "Edge.Cuts") (width 0.15))
 (segment (start 24.9276 28.1695) (end 26.1976 28.1695) (width 0.2) (layer "F.Cu") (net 2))
 (segment (start 29.2456 28.1695) (end 30.55 28.1695) (width 0.2) (layer "F.Cu") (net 2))
 (segment (start 30.485475 25.462775) (end 32.243297 25.462775) (width 0.2) (layer "F.Cu") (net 26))
 (segment (start 32.812533 26.032011) (end 32.812533 28.900033) (width 0.2) (layer "F.Cu") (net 26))
 (segment (start 28.6766 31.657) (end 28.6766 31.396842) (width 0.2) (layer "F.Cu") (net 26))
 (segment (start 33.725 29.8125) (end 32.914725 30.622775) (width 0.2) (layer "F.Cu") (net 26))
 (segment (start 28.6766 31.396842) (end 27.782533 30.502775) (width 0.2) (layer "F.Cu") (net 26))
 (segment (start 32.812533 28.900033) (end 33.725 29.8125) (width 0.2) (layer "F.Cu") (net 26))
 (segment (start 24.192533 30.077926) (end 24.800629 30.686022) (width 0.2) (layer "F.Cu") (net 26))
 (segment (start 23.6695 27.8526) (end 23.6695 28.3345) (width 0.2) (layer "F.Cu") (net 26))
 (segment (start 29.572533 30.622775) (end 28.6766 31.518708) (width 0.2) (layer "F.Cu") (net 26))
 (segment (start 27.7216 28.602) (end 27.7216 30.441842) (width 0.2) (layer "F.Cu") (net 26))
 (segment (start 25.32145 24.49875) (end 25.32145 26.20065) (width 0.2) (layer "F.Cu") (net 26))
 (segment (start 24.9276 26.5945) (end 23.6695 27.8526) (width 0.2) (layer "F.Cu") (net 26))
 (segment (start 30.12145 24.49875) (end 30.12145 25.09875) (width 0.2) (layer "F.Cu") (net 26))
 (segment (start 32.914725 30.622775) (end 29.572533 30.622775) (width 0.2) (layer "F.Cu") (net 26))
 (segment (start 30.12145 25.09875) (end 30.485475 25.462775) (width 0.2) (layer "F.Cu") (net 26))
 (segment (start 32.243297 25.462775) (end 32.812533 26.032011) (width 0.2) (layer "F.Cu") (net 26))
 (segment (start 27.599286 30.686022) (end 27.782533 30.502775) (width 0.2) (layer "F.Cu") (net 26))
 (segment (start 25.32145 26.20065) (end 24.9276 26.5945) (width 0.2) (layer "F.Cu") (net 26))
 (segment (start 24.800629 30.686022) (end 27.599286 30.686022) (width 0.2) (layer "F.Cu") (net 26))
 (segment (start 23.6695 28.3345) (end 24.192533 28.857533) (width 0.2) (layer "F.Cu") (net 26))
 (segment (start 27.7216 30.441842) (end 27.782533 30.502775) (width 0.2) (layer "F.Cu") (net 26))
 (segment (start 28.6766 31.518708) (end 28.6766 31.657) (width 0.2) (layer "F.Cu") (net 26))
 (segment (start 24.192533 28.857533) (end 24.192533 30.077926) (width 0.2) (layer "F.Cu") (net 26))
 (segment (start 23.852533 37.152775) (end 23.852533 36.602775) (width 0.2) (layer "F.Cu") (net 40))
 (segment (start 26.5716 25.508) (end 26.5716 25.595497) (width 0.2) (layer "F.Cu") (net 40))
 (segment (start 23.852533 36.602775) (end 24.172533 36.282775) (width 0.2) (layer "F.Cu") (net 40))
 (segment locked (start 26.5716 25.508) (end 26.9716 25.108) (width 0.2) (layer "F.Cu") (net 40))
 (segment locked (start 27.9716 24.73) (end 27.9716 25.593898) (width 0.2) (layer "F.Cu") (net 40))
 (segment locked (start 26.9716 25.108) (end 26.9716 24.5) (width 0.2) (layer "F.Cu") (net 40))
 (via (at 24.172533 36.282775) (size 0.6) (drill 0.33) (layers "F.Cu" "B.Cu") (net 40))
 (via (at 26.5716 25.595497) (size 0.6) (drill 0.33) (layers "F.Cu" "B.Cu") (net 40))
 (via (at 27.972533 25.582775) (size 0.6) (drill 0.33) (layers "F.Cu" "B.Cu") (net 40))
 (segment locked (start 26.5716 25.595497) (end 27.969999 25.595497) (width 0.2) (layer "B.Cu") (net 40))
 (segment (start 24.172533 36.282775) (end 24.172533 29.748773) (width 0.2) (layer "B.Cu") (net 40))
 (segment (start 26.422533 25.744564) (end 26.5716 25.595497) (width 0.2) (layer "B.Cu") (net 40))
 (segment (start 26.422533 27.498773) (end 26.422533 25.744564) (width 0.2) (layer "B.Cu") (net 40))
 (segment (start 24.172533 29.748773) (end 26.422533 27.498773) (width 0.2) (layer "B.Cu") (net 40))
 (segment locked (start 27.0676 25.947335) (end 27.2176 25.797335) (width 0.2) (layer "F.Cu") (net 41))
 (segment locked (start 28.569511 25.347171) (end 28.4716 25.24926) (width 0.2) (layer "F.Cu") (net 41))
 (segment (start 27.0676 27.232) (end 27.0676 27.389966) (width 0.2) (layer "F.Cu") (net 41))
 (segment locked (start 27.0676 27.232) (end 27.0676 25.947335) (width 0.2) (layer "F.Cu") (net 41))
 (segment locked (start 28.4716 25.24926) (end 28.4716 24.6) (width 0.2) (layer "F.Cu") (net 41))
 (segment locked (start 27.2176 25.797335) (end 27.2176 25.442) (width 0.2) (layer "F.Cu") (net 41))
 (segment (start 25.012533 36.172775) (end 25.012533 37.092775) (width 0.2) (layer "F.Cu") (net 41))
 (segment locked (start 28.569511 25.940089) (end 28.569511 25.347171) (width 0.2) (layer "F.Cu") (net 41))
 (segment locked (start 27.4716 25.188) (end 27.4716 24.6) (width 0.2) (layer "F.Cu") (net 41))
 (segment (start 27.0676 27.389966) (end 27.081967 27.404333) (width 0.2) (layer "F.Cu") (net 41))
 (segment (start 25.012533 37.092775) (end 24.952533 37.152775) (width 0.2) (layer "F.Cu") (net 41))
 (segment locked (start 27.2176 25.442) (end 27.4716 25.188) (width 0.2) (layer "F.Cu") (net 41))
 (segment locked (start 28.4076 26.102) (end 28.569511 25.940089) (width 0.2) (layer "F.Cu") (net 41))
 (segment locked (start 28.4076 27.212) (end 28.4076 26.102) (width 0.2) (layer "F.Cu") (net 41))
 (via (at 27.081967 27.404333) (size 0.6) (drill 0.33) (layers "F.Cu" "B.Cu") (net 41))
 (via (at 25.012533 36.172775) (size 0.6) (drill 0.33) (layers "F.Cu" "B.Cu") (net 41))
 (via (at 28.3211 27.112775) (size 0.6) (drill 0.33) (layers "F.Cu" "B.Cu") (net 41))
 (segment (start 24.582533 35.742775) (end 25.012533 36.172775) (width 0.2) (layer "B.Cu") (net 41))
 (segment (start 24.582533 29.903767) (end 24.582533 35.742775) (width 0.2) (layer "B.Cu") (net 41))
 (segment (start 28.012533 27.404333) (end 27.081967 27.404333) (width 0.2) (layer "B.Cu") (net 41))
 (segment (start 28.3211 27.112775) (end 28.012533 27.404333) (width 0.2) (layer "B.Cu") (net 41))
 (segment (start 27.081967 27.404333) (end 24.582533 29.903767) (width 0.2) (layer "B.Cu") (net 41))
 (segment (start 30.55 26.5945) (end 31.606 26.5945) (width 0.2) (layer "F.Cu") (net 23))
 (segment (start 31.606 26.5945) (end 31.766 26.4345) (width 0.2) (layer "F.Cu") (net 23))
 (segment (start 25.97145 24.49875) (end 25.97145 26.36835) (width 0.2) (layer "F.Cu") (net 29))
 (segment (start 25.97145 26.36835) (end 26.1976 26.5945) (width 0.2) (layer "F.Cu") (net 29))
 (segment (start 28.97145 24.49875) (end 28.97145 26.32035) (width 0.2) (layer "F.Cu") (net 30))
 (segment (start 28.97145 26.32035) (end 29.2456 26.5945) (width 0.2) (layer "F.Cu") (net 30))
 (segment (start 21.7 29.8125) (end 23.3 29.8125) (width 0.2) (layer "F.Cu") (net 28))
 (segment (start 26.7666 30.187) (end 26.667089 30.286511) (width 0.2) (layer "F.Cu") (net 25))
 (segment (start 26.97212 28.152458) (end 26.97212 29.25148) (width 0.2) (layer "F.Cu") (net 25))
 (segment (start 27.7216 27.683708) (end 27.402819 28.002489) (width 0.2) (layer "F.Cu") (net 25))
 (segment (start 26.667089 30.286511) (end 24.966111 30.286511) (width 0.2) (layer "F.Cu") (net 25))
 (segment (start 27.7216 26.402) (end 27.7216 27.683708) (width 0.2) (layer "F.Cu") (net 25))
 (segment (start 24.966111 30.286511) (end 24.8666 30.187) (width 0.2) (layer "F.Cu") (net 25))
 (segment (start 26.7666 29.457) (end 26.7666 30.187) (width 0.2) (layer "F.Cu") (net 25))
 (segment (start 27.122089 28.002489) (end 26.97212 28.152458) (width 0.2) (layer "F.Cu") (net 25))
 (segment (start 24.8666 30.187) (end 24.8666 29.457) (width 0.2) (layer "F.Cu") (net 25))
 (segment (start 27.402819 28.002489) (end 27.122089 28.002489) (width 0.2) (layer "F.Cu") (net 25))
 (segment (start 26.97212 29.25148) (end 26.7666 29.457) (width 0.2) (layer "F.Cu") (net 25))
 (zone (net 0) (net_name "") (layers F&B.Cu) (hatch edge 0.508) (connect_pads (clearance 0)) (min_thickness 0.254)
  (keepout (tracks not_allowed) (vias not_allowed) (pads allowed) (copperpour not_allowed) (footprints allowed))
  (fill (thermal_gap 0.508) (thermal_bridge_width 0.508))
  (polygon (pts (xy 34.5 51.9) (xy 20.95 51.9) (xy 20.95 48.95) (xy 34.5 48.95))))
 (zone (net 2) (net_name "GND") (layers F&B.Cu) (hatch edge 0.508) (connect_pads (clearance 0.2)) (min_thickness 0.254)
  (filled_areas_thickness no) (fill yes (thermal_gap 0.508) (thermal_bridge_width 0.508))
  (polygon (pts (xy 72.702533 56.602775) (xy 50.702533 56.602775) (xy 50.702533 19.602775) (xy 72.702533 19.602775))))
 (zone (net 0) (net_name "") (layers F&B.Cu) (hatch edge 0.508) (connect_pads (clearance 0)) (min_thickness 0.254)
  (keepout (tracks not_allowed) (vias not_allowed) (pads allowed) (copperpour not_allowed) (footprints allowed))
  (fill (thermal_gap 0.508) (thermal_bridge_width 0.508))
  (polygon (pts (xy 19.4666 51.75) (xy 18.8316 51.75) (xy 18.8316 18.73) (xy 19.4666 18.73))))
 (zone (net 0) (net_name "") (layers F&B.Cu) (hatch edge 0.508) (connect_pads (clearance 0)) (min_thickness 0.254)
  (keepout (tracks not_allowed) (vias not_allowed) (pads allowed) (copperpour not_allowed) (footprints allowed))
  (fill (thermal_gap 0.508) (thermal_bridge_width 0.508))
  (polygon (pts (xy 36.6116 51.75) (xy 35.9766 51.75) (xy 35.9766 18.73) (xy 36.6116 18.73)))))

